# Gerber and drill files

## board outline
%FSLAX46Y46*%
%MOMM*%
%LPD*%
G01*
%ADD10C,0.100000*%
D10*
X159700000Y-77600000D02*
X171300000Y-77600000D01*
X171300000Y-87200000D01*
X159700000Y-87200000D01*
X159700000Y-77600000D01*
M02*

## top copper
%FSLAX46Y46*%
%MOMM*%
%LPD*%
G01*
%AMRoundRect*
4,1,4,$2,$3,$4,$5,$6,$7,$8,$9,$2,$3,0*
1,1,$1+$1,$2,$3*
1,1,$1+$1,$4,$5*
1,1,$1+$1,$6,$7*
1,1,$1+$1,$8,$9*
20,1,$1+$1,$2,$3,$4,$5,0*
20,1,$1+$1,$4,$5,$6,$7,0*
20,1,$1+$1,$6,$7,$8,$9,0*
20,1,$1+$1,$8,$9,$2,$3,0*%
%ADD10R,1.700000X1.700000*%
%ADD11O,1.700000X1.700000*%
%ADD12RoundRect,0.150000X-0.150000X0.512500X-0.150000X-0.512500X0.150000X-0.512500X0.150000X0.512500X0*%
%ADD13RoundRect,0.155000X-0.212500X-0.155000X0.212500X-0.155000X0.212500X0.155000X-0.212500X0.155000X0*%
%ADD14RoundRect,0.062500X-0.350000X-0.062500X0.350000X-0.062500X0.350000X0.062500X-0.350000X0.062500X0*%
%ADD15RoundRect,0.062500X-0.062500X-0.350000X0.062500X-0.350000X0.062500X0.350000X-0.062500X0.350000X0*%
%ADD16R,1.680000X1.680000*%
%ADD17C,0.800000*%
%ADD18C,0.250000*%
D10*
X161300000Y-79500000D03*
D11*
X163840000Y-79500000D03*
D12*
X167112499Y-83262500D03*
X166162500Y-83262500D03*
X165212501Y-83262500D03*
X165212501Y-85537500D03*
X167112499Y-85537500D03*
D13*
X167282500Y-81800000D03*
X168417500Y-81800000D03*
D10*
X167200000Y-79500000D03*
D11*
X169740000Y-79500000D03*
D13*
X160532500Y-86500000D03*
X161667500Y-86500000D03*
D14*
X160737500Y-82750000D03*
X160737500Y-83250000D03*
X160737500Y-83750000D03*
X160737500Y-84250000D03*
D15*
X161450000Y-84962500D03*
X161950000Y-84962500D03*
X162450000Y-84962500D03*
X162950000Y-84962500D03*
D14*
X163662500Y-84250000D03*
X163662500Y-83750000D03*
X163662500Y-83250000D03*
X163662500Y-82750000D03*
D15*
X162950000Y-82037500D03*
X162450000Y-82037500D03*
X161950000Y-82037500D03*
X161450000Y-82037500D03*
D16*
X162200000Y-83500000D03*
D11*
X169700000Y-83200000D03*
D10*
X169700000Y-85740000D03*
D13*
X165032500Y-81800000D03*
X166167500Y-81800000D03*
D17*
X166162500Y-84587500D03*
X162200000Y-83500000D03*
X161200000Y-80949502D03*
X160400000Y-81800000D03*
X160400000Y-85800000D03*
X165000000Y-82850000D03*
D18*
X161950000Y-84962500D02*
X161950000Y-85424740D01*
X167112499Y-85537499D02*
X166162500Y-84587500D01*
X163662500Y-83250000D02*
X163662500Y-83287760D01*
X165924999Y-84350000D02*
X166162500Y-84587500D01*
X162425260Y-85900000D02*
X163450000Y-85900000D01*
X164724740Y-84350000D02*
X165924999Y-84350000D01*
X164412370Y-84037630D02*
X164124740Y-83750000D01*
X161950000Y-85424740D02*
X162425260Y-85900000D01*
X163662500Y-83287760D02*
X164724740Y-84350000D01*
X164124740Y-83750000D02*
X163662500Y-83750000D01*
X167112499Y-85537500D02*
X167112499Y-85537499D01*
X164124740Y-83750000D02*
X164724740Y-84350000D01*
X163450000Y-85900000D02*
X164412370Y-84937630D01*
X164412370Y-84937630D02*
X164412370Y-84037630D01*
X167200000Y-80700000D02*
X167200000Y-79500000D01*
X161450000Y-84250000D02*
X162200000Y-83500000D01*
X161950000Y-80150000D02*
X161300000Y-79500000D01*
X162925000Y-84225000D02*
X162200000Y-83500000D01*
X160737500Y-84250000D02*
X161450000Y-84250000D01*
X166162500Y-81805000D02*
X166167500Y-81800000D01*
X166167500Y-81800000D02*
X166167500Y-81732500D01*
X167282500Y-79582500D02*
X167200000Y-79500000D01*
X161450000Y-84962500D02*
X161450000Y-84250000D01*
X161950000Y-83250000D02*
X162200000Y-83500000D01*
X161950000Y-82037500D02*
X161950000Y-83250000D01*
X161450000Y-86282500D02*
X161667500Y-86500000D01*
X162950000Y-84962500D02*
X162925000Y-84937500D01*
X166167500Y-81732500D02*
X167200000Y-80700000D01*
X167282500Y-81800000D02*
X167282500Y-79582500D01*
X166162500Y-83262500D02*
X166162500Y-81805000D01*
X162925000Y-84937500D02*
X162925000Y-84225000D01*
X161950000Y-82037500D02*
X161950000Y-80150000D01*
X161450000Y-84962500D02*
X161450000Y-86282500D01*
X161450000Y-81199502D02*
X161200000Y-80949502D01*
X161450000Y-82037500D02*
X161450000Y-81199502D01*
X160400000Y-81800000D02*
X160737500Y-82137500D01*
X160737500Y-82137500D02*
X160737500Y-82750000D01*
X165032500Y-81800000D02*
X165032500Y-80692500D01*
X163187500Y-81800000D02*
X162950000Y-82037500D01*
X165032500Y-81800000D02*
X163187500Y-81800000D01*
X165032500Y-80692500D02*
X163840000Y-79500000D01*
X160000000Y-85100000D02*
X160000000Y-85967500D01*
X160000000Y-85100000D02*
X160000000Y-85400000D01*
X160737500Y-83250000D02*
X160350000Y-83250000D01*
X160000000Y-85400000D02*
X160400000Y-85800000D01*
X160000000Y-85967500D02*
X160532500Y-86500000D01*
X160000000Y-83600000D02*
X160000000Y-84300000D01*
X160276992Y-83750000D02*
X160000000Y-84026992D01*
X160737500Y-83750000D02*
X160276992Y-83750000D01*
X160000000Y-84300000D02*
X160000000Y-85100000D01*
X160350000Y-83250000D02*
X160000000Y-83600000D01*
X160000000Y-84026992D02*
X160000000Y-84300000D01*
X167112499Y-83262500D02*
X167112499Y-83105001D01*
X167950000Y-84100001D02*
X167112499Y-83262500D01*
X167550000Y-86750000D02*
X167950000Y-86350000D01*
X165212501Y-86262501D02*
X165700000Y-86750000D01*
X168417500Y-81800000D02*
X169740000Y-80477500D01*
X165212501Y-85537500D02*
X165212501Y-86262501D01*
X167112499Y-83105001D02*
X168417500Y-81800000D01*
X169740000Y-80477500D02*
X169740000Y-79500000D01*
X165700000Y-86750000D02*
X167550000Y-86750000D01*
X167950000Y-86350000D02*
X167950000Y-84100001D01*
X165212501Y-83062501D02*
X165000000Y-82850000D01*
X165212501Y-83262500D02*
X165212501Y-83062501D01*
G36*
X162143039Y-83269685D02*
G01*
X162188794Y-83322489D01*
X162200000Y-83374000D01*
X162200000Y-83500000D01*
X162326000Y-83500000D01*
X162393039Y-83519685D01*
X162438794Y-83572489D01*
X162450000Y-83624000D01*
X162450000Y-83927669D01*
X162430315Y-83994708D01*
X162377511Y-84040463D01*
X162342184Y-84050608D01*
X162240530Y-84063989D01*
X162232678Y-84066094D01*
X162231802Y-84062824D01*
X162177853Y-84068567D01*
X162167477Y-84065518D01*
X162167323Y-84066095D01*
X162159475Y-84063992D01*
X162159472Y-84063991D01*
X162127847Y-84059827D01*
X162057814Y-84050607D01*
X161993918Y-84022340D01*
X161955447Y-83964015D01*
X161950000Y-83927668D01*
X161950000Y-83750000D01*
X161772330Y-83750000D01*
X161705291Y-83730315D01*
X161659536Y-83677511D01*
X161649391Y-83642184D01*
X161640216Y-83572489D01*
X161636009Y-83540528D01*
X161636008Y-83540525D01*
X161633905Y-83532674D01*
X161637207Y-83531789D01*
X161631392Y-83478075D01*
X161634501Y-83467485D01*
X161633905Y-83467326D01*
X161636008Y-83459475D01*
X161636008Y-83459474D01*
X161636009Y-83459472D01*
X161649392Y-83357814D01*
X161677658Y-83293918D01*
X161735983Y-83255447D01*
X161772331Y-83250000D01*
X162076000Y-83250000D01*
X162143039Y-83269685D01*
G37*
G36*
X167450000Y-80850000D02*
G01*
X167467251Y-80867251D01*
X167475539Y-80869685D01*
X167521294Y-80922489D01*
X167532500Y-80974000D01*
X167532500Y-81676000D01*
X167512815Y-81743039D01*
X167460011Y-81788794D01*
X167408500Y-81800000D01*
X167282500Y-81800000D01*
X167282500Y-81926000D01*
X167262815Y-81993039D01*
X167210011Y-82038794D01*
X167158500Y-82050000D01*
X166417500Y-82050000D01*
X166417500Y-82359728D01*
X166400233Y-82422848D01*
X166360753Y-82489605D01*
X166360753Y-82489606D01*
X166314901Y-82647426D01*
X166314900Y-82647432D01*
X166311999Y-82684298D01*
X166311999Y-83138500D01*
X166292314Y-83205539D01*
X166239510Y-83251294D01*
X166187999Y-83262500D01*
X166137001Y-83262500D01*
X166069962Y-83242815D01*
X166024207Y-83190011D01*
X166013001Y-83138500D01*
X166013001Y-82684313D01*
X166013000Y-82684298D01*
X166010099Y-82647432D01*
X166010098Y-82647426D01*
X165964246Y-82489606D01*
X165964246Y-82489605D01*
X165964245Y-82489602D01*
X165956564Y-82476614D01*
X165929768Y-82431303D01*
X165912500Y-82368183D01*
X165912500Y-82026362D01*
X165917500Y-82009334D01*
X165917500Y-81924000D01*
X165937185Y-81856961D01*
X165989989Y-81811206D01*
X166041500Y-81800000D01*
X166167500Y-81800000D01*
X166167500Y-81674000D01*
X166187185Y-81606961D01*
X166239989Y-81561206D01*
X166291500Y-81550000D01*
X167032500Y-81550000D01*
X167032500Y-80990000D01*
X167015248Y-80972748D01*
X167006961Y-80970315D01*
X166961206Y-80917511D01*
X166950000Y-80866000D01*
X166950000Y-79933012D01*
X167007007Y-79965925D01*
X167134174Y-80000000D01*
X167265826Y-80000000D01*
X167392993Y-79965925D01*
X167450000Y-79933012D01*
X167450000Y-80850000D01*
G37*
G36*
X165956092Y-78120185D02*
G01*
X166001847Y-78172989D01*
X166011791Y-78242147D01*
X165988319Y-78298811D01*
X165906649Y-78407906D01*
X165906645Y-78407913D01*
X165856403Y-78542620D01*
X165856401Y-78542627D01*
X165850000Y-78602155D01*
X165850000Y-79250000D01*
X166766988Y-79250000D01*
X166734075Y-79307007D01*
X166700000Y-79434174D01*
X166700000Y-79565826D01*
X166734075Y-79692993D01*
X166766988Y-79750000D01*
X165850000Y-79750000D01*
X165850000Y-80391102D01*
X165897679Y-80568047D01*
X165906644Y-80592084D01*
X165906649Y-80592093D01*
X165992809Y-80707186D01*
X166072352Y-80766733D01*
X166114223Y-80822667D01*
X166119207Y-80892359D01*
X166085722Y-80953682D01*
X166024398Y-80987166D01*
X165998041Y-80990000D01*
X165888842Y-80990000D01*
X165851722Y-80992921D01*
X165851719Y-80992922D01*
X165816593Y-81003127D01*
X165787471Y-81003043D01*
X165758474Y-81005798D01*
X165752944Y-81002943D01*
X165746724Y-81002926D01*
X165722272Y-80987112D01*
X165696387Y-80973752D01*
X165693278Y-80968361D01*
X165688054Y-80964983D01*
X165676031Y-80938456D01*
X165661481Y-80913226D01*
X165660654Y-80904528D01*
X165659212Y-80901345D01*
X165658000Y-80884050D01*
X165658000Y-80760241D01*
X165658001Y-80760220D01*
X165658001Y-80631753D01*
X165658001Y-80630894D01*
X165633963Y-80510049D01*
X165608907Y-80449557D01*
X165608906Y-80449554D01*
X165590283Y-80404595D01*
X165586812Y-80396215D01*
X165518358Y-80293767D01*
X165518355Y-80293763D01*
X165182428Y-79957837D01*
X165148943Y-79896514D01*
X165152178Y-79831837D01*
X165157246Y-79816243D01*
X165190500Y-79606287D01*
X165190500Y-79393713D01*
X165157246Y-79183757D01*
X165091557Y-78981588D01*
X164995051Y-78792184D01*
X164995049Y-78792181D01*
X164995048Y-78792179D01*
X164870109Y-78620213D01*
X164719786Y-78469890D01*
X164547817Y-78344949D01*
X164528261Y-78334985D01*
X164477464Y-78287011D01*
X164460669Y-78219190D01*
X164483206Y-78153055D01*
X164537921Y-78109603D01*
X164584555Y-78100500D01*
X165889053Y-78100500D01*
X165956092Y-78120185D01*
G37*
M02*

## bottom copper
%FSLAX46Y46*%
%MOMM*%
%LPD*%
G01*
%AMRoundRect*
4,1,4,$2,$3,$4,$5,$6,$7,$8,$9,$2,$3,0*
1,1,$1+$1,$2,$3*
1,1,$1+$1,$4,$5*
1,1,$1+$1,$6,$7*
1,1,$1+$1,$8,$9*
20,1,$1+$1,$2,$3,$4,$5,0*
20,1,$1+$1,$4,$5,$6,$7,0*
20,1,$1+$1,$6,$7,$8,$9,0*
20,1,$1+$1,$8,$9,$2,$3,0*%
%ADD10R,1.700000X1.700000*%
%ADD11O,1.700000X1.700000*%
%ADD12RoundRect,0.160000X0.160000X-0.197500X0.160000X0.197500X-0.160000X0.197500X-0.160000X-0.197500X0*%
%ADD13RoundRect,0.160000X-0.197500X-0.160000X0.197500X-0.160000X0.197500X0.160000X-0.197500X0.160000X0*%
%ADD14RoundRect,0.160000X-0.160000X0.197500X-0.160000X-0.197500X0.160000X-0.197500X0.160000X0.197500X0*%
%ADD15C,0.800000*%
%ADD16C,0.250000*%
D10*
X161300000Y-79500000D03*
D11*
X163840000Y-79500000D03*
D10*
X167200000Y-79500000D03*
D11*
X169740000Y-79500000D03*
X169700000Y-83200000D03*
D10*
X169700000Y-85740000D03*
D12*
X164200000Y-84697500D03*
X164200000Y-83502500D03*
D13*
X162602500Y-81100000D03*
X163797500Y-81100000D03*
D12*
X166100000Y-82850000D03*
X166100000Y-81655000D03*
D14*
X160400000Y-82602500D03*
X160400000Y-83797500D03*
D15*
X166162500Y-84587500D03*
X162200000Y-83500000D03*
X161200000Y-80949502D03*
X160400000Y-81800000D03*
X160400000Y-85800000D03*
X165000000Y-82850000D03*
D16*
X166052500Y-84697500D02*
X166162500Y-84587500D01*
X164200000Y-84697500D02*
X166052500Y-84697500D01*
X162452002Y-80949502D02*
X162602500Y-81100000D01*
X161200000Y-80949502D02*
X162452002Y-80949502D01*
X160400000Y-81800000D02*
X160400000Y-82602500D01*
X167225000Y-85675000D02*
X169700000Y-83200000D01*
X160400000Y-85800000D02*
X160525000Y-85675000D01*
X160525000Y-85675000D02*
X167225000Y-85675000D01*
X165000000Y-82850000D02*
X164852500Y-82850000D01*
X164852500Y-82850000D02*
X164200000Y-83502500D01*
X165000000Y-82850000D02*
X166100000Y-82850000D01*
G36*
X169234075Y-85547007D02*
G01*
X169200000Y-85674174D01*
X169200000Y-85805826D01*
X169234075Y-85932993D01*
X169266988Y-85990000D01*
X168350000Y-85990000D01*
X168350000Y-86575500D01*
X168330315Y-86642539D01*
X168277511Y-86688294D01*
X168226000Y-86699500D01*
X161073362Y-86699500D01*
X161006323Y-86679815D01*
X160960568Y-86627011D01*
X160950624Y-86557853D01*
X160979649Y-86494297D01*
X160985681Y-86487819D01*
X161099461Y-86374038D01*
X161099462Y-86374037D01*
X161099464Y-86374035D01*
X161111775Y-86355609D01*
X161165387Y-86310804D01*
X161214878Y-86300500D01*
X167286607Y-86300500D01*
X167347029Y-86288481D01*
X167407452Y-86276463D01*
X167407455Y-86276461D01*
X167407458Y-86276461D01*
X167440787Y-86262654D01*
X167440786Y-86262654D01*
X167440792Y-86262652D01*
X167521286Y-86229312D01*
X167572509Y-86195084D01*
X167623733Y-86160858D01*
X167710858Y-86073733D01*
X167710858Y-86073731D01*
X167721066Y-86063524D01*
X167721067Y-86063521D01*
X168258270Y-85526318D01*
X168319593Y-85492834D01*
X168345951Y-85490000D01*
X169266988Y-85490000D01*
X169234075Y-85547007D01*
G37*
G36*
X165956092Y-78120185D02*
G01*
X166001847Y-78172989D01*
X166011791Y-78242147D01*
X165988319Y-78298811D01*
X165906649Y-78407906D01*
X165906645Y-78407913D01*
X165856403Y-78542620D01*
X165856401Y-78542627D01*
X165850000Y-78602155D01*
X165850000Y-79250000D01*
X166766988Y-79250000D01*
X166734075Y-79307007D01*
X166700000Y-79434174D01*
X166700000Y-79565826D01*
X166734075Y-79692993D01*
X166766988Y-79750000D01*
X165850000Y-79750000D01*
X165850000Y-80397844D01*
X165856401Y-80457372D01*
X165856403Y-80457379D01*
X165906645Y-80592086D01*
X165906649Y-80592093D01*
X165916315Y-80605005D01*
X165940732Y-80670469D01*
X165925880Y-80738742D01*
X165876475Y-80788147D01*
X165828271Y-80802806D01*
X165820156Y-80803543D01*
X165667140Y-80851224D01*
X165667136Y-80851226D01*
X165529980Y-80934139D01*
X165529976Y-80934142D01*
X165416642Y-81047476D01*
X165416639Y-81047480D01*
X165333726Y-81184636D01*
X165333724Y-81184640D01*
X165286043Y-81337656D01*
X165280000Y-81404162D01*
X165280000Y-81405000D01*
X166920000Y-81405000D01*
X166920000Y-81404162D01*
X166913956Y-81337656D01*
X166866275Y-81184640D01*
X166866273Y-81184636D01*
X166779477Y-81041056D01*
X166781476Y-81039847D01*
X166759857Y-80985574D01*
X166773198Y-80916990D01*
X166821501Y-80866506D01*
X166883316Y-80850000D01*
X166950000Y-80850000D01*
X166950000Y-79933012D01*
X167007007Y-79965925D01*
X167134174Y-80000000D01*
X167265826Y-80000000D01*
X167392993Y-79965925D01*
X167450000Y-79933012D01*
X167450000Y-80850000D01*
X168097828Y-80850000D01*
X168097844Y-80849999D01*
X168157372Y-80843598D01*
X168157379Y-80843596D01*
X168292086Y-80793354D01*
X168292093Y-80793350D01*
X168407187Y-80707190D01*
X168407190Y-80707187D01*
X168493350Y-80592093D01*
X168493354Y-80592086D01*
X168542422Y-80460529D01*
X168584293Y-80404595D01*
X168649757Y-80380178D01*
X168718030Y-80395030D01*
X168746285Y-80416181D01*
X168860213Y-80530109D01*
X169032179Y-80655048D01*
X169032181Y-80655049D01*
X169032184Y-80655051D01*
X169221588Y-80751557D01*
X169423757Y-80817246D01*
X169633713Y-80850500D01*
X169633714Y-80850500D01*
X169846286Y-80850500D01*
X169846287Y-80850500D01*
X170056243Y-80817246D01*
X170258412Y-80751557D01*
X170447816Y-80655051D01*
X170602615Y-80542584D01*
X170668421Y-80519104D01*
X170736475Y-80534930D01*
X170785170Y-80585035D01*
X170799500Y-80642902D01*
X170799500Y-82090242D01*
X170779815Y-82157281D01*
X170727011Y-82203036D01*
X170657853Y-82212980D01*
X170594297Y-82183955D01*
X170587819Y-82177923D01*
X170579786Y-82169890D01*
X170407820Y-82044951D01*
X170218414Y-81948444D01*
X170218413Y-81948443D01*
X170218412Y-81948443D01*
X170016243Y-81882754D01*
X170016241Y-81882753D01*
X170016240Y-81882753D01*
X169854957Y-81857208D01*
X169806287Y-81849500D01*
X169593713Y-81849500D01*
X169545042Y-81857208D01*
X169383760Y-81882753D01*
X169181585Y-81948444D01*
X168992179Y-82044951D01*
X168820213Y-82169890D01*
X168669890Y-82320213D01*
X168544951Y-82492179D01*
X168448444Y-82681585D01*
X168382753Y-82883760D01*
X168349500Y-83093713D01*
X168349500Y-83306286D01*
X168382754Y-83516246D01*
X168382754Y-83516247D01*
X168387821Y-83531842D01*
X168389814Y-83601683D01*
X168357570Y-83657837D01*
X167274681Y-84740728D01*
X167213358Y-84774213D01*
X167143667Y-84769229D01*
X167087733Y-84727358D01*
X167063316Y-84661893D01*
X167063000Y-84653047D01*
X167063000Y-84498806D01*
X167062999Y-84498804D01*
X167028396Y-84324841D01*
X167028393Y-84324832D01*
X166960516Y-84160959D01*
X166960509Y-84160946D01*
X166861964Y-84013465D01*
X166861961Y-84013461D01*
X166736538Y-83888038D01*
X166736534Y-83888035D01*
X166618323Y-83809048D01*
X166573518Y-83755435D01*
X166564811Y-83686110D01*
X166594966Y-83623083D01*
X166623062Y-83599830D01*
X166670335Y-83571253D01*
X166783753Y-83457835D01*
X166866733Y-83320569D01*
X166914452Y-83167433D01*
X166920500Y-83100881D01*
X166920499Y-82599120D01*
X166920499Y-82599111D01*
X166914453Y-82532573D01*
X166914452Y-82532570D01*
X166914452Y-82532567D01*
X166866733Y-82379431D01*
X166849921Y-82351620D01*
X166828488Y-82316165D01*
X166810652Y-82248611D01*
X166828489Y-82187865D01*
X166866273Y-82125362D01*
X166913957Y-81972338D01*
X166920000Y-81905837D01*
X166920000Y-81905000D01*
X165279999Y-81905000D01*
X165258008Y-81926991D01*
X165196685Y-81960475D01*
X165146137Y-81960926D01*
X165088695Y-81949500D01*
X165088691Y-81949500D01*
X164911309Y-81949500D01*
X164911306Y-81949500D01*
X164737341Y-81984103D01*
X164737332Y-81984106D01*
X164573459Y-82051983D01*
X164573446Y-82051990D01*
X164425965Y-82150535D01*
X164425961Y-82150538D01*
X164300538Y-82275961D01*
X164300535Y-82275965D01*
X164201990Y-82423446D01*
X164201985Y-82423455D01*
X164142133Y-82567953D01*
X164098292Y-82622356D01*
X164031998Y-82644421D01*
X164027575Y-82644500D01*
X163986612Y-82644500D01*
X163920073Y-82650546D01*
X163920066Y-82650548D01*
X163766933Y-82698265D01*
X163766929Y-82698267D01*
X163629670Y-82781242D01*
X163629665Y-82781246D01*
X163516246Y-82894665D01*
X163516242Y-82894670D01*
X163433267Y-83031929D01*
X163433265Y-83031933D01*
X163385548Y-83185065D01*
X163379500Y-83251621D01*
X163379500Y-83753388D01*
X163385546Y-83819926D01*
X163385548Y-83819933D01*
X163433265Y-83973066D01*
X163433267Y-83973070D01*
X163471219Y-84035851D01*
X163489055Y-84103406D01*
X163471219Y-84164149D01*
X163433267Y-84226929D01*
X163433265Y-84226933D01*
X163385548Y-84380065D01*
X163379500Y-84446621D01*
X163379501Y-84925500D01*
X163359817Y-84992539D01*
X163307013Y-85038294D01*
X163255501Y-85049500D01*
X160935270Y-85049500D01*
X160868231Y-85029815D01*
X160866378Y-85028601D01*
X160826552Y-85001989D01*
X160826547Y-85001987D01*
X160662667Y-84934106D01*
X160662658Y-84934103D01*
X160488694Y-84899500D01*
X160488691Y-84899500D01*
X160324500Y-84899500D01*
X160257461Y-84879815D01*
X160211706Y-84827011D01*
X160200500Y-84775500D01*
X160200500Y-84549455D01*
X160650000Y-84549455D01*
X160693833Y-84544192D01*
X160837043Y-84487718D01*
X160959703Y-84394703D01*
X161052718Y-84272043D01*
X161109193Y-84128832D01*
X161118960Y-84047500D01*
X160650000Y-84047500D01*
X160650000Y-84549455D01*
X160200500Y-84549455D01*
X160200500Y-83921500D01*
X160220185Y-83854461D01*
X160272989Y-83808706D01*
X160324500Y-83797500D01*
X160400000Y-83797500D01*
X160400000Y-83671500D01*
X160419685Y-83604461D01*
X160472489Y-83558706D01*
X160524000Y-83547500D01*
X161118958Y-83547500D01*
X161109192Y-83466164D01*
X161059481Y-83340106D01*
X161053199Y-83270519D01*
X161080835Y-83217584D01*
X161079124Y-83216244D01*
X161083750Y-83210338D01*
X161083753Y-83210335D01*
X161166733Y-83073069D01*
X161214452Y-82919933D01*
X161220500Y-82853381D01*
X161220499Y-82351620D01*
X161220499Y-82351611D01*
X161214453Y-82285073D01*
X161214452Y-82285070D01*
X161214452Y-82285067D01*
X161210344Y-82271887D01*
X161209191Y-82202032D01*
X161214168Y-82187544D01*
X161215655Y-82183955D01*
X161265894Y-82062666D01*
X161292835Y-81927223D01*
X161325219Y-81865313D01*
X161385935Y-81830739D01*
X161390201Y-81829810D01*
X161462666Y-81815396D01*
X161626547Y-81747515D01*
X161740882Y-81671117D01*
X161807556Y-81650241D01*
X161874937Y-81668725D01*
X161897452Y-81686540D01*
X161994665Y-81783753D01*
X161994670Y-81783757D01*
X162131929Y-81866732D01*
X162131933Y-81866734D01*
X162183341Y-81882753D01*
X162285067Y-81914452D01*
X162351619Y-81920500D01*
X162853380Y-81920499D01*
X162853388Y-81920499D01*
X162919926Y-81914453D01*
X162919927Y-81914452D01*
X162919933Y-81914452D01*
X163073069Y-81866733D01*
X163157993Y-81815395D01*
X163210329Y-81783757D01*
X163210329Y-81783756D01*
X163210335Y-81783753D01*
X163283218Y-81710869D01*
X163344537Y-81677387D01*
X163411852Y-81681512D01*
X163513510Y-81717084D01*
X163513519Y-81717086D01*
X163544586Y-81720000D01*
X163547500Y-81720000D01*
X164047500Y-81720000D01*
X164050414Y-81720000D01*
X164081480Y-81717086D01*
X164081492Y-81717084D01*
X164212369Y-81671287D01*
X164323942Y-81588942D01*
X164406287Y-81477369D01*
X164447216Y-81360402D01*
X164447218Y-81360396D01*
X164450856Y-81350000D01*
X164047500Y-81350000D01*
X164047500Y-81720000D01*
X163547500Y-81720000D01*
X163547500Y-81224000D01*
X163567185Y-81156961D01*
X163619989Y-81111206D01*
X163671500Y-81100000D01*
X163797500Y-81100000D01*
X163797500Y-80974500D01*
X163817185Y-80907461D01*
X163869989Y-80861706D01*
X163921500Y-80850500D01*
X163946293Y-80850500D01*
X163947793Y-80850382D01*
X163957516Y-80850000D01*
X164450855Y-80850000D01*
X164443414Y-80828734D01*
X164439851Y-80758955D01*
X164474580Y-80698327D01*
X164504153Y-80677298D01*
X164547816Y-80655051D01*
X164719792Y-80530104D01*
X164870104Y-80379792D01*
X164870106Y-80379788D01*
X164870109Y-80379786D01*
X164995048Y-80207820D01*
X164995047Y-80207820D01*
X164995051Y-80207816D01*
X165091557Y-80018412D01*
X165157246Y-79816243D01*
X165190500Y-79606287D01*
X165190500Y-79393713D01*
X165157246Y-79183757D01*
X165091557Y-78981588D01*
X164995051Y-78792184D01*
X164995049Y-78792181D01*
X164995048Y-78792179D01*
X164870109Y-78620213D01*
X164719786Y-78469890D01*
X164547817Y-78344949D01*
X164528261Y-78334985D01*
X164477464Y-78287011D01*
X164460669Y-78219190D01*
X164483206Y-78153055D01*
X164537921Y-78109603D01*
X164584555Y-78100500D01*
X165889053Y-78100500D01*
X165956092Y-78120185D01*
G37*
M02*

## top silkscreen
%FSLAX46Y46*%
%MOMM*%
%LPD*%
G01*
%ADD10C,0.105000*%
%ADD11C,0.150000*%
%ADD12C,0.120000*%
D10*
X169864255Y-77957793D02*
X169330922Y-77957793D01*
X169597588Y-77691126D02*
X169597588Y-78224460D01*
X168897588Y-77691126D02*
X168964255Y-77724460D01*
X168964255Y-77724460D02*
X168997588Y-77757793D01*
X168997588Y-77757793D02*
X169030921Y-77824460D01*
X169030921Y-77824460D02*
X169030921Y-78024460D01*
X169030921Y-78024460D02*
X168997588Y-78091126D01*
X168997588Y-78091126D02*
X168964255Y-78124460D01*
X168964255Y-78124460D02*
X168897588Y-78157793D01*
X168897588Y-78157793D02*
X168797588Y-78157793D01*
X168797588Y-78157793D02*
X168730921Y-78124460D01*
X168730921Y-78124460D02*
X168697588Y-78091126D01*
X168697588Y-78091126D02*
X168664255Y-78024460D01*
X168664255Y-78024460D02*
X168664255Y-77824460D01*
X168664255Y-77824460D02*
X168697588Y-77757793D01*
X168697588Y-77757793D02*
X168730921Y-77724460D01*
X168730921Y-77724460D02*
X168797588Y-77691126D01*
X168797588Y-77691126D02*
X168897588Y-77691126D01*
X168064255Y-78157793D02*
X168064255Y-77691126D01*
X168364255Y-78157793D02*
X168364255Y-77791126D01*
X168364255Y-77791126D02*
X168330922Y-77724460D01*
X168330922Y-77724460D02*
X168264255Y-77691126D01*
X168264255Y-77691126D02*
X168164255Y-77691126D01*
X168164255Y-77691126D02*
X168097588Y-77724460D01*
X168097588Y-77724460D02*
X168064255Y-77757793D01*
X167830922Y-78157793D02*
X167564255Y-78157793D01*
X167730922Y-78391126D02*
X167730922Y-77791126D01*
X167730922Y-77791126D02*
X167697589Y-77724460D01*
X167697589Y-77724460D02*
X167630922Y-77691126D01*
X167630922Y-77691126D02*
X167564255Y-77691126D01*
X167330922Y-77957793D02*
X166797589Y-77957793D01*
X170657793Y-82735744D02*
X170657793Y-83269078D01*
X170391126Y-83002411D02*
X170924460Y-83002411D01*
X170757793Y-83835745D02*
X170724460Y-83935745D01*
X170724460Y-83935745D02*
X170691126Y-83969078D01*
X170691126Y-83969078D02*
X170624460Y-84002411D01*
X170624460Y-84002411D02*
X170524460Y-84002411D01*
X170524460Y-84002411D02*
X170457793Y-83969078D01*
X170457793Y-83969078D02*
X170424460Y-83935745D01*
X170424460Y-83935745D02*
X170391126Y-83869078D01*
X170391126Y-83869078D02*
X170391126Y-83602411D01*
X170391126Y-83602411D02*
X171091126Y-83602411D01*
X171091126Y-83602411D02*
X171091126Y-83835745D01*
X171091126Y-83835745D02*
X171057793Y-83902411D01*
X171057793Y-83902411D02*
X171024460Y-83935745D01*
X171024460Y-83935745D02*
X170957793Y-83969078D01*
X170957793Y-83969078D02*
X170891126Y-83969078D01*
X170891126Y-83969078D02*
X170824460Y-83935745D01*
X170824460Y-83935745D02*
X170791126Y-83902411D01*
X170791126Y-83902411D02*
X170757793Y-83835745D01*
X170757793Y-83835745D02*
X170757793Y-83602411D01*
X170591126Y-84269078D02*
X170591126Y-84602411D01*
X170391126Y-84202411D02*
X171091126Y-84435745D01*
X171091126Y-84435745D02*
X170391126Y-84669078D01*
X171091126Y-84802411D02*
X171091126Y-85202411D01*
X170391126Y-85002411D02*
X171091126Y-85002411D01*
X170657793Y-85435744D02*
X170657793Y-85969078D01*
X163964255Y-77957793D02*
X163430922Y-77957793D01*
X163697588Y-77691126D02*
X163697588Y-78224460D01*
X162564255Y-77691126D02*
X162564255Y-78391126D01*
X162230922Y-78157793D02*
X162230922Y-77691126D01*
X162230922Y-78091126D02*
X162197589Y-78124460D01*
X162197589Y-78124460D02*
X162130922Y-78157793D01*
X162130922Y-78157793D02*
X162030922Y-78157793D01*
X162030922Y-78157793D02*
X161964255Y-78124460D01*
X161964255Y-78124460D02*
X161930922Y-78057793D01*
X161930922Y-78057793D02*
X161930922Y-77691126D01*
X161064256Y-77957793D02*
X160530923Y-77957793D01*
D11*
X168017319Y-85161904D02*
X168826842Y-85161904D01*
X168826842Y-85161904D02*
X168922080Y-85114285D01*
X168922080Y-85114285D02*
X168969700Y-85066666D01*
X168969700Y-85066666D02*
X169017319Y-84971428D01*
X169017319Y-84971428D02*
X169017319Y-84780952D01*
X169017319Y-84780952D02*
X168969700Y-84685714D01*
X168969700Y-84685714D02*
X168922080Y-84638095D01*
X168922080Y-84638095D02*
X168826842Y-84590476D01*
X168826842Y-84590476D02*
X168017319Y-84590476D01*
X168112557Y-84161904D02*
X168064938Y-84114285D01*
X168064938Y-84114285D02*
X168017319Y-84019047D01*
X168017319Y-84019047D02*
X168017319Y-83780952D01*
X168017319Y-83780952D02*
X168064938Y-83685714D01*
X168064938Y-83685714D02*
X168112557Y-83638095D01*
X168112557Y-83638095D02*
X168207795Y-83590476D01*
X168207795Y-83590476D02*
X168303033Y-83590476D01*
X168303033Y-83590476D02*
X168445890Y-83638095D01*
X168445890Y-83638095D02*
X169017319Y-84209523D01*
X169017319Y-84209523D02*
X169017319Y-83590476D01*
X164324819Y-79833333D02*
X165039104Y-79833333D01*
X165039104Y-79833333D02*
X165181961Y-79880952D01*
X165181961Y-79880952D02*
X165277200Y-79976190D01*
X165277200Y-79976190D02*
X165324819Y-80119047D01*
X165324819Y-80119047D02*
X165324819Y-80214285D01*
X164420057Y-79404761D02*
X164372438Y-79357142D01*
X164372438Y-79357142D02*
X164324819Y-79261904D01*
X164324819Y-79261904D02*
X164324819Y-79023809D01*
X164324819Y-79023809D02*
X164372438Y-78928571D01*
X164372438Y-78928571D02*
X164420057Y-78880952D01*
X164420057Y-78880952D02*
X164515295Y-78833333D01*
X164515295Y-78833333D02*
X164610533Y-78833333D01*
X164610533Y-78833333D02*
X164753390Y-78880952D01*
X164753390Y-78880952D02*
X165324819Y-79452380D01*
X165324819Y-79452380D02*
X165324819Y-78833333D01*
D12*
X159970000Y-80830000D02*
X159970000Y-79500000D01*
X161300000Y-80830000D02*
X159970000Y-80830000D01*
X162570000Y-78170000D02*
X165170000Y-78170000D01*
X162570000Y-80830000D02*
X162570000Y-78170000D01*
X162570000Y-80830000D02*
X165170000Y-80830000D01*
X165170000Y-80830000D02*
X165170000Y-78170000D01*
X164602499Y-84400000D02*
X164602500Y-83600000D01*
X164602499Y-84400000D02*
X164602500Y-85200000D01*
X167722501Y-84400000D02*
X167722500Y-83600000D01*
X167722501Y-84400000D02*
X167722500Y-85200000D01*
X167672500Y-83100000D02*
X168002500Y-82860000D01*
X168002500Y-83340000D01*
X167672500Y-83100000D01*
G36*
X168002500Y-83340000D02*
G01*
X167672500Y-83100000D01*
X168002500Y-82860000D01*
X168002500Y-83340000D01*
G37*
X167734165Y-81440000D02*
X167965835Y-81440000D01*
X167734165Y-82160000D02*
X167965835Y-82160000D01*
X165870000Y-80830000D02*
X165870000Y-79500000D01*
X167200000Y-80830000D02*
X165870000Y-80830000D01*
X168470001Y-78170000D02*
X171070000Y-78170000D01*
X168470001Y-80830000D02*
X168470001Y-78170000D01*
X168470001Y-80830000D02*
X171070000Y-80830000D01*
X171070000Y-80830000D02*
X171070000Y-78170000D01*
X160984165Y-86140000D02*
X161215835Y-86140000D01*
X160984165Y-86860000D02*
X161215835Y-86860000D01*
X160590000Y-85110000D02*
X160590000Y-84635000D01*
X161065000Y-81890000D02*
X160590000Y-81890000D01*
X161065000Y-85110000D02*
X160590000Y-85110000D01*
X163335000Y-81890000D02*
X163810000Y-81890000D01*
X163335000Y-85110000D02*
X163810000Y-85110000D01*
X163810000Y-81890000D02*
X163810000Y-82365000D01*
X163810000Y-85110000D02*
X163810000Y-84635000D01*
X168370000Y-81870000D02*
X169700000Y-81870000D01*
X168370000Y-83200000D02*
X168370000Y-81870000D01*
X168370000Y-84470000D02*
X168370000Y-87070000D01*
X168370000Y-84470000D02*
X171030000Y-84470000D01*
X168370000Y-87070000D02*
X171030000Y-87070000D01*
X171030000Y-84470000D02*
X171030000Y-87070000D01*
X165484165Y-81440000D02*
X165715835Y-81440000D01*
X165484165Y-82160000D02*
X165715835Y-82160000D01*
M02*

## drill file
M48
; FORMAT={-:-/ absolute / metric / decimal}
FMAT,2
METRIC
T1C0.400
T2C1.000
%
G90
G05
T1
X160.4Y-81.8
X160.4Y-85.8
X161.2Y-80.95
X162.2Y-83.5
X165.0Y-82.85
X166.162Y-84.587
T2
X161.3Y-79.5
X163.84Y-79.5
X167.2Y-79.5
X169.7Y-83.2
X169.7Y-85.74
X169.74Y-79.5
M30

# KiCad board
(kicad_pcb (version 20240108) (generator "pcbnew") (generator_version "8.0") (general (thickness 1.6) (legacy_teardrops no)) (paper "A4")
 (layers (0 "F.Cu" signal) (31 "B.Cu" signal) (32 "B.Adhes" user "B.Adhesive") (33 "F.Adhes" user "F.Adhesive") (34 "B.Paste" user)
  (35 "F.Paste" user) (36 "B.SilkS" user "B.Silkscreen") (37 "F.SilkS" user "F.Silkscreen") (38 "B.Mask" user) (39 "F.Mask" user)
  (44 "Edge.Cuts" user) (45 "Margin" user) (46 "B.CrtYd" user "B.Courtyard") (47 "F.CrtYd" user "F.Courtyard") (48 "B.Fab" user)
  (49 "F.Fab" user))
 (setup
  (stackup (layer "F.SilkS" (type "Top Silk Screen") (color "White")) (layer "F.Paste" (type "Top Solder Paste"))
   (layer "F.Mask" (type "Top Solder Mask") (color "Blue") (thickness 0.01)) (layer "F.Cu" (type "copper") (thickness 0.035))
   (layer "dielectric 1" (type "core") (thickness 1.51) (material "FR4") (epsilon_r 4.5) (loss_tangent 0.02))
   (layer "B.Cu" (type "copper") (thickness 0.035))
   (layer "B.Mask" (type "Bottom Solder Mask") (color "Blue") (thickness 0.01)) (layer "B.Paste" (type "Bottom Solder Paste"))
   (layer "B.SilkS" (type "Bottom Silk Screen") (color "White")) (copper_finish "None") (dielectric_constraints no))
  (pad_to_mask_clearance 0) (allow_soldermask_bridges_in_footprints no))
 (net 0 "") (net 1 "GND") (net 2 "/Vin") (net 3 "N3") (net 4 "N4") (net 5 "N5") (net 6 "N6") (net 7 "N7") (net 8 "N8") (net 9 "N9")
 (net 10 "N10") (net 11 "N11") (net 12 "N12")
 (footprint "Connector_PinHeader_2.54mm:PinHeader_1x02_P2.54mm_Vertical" (layer "F.Cu") (at 161.3 79.5 90)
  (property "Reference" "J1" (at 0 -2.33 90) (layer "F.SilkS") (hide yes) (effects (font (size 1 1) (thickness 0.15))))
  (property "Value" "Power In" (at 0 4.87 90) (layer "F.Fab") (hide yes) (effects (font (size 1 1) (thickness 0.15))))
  (fp_line (start -1.33 -1.33) (end 0 -1.33) (stroke (width 0.12) (type solid)) (layer "F.SilkS"))
  (fp_line (start -1.33 0) (end -1.33 -1.33) (stroke (width 0.12) (type solid)) (layer "F.SilkS"))
  (fp_line (start 1.33 1.27) (end 1.33 3.87) (stroke (width 0.12) (type solid)) (layer "F.SilkS"))
  (fp_line (start -1.33 1.27) (end 1.33 1.27) (stroke (width 0.12) (type solid)) (layer "F.SilkS"))
  (fp_line (start -1.33 1.27) (end -1.33 3.87) (stroke (width 0.12) (type solid)) (layer "F.SilkS"))
  (fp_line (start -1.33 3.87) (end 1.33 3.87) (stroke (width 0.12) (type solid)) (layer "F.SilkS"))
  (pad "1" thru_hole rect (at 0 0 90) (size 1.7 1.7) (drill 1) (layers "*.Cu" "*.Mask") (remove_unused_layers no) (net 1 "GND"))
  (pad "2" thru_hole oval (at 0 2.54 90) (size 1.7 1.7) (drill 1) (layers "*.Cu" "*.Mask") (remove_unused_layers no) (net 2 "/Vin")))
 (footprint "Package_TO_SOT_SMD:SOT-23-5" (layer "F.Cu") (at 166.1625 84.4 -90)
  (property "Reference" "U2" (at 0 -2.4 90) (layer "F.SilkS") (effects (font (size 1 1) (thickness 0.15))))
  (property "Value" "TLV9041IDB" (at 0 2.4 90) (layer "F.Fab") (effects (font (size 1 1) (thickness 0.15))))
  (fp_line (start 0 1.560001) (end -0.8 1.56) (stroke (width 0.12) (type solid)) (layer "F.SilkS"))
  (fp_line (start 0 1.560001) (end 0.8 1.56) (stroke (width 0.12) (type solid)) (layer "F.SilkS"))
  (fp_line (start 0 -1.560001) (end -0.8 -1.56) (stroke (width 0.12) (type solid)) (layer "F.SilkS"))
  (fp_line (start 0 -1.560001) (end 0.8 -1.56) (stroke (width 0.12) (type solid)) (layer "F.SilkS"))
  (fp_poly
   (pts (xy -1.3 -1.51) (xy -1.54 -1.84) (xy -1.06 -1.84) (xy -1.3 -1.51)) (stroke (width 0.12) (type solid)) (fill solid) (layer "F.SilkS"))
  (pad "1" smd roundrect (at -1.1375 -0.949999 270) (size 1.325 0.6) (layers "F.Cu" "F.Paste" "F.Mask") (roundrect_rratio 0.25) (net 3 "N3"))
  (pad "2" smd roundrect (at -1.1375 0 270) (size 1.325 0.6) (layers "F.Cu" "F.Paste" "F.Mask") (roundrect_rratio 0.25) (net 1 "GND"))
  (pad "3" smd roundrect (at -1.1375 0.949999 270) (size 1.325 0.6) (layers "F.Cu" "F.Paste" "F.Mask") (roundrect_rratio 0.25) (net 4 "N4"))
  (pad "4" smd roundrect (at 1.1375 0.949999 270) (size 1.325 0.6) (layers "F.Cu" "F.Paste" "F.Mask") (roundrect_rratio 0.25) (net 3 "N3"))
  (pad "5" smd roundrect (at 1.1375 -0.949999 270) (size 1.325 0.6) (layers "F.Cu" "F.Paste" "F.Mask") (roundrect_rratio 0.25) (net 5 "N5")))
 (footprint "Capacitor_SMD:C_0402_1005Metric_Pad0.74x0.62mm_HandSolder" (layer "F.Cu") (at 167.85 81.8)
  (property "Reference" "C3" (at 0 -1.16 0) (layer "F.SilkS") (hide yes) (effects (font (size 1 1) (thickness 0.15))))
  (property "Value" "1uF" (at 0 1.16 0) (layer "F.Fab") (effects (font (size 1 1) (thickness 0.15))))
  (fp_line (start -0.115835 -0.36) (end 0.115835 -0.36) (stroke (width 0.12) (type solid)) (layer "F.SilkS"))
  (fp_line (start -0.115835 0.36) (end 0.115835 0.36) (stroke (width 0.12) (type solid)) (layer "F.SilkS"))
  (pad "1" smd roundrect (at -0.5675 0) (size 0.735 0.62) (layers "F.Cu" "F.Paste" "F.Mask") (roundrect_rratio 0.25) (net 1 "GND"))
  (pad "2" smd roundrect (at 0.5675 0) (size 0.735 0.62) (layers "F.Cu" "F.Paste" "F.Mask") (roundrect_rratio 0.25) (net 3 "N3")))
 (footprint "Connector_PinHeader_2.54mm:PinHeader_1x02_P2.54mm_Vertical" (layer "F.Cu") (at 167.2 79.5 90)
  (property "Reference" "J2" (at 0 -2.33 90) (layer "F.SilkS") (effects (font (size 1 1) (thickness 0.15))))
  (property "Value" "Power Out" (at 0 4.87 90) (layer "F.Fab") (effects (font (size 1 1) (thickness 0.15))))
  (fp_line (start -1.33 -1.33) (end 0 -1.33) (stroke (width 0.12) (type solid)) (layer "F.SilkS"))
  (fp_line (start -1.33 0) (end -1.33 -1.33) (stroke (width 0.12) (type solid)) (layer "F.SilkS"))
  (fp_line (start 1.33 1.270001) (end 1.33 3.87) (stroke (width 0.12) (type solid)) (layer "F.SilkS"))
  (fp_line (start -1.33 1.270001) (end 1.33 1.270001) (stroke (width 0.12) (type solid)) (layer "F.SilkS"))
  (fp_line (start -1.33 1.270001) (end -1.33 3.87) (stroke (width 0.12) (type solid)) (layer "F.SilkS"))
  (fp_line (start -1.33 3.87) (end 1.33 3.87) (stroke (width 0.12) (type solid)) (layer "F.SilkS"))
  (pad "1" thru_hole rect (at 0 0 90) (size 1.7 1.7) (drill 1) (layers "*.Cu" "*.Mask") (remove_unused_layers no) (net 1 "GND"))
  (pad "2" thru_hole oval (at 0 2.54 90) (size 1.7 1.7) (drill 1) (layers "*.Cu" "*.Mask") (remove_unused_layers no) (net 3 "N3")))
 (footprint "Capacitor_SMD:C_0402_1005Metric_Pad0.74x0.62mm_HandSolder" (layer "F.Cu") (at 161.1 86.5)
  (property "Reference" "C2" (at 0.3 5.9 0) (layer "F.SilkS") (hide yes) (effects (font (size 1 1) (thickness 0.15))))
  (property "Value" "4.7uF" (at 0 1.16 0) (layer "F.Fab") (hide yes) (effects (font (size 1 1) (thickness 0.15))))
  (fp_line (start -0.115835 -0.36) (end 0.115835 -0.36) (stroke (width 0.12) (type solid)) (layer "F.SilkS"))
  (fp_line (start -0.115835 0.36) (end 0.115835 0.36) (stroke (width 0.12) (type solid)) (layer "F.SilkS"))
  (pad "1" smd roundrect (at -0.5675 0) (size 0.735 0.62) (layers "F.Cu" "F.Paste" "F.Mask") (roundrect_rratio 0.25) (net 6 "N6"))
  (pad "2" smd roundrect (at 0.5675 0) (size 0.735 0.62) (layers "F.Cu" "F.Paste" "F.Mask") (roundrect_rratio 0.25) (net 1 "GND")))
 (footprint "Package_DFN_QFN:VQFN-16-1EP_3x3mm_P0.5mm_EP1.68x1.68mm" (layer "F.Cu") (at 162.2 83.5)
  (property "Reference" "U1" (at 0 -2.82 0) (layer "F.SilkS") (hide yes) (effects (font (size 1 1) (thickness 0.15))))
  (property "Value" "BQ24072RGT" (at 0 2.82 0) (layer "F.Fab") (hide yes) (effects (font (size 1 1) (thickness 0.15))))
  (fp_line (start -1.61 1.61) (end -1.61 1.135) (stroke (width 0.12) (type solid)) (layer "F.SilkS"))
  (fp_line (start -1.135 -1.61) (end -1.61 -1.61) (stroke (width 0.12) (type solid)) (layer "F.SilkS"))
  (fp_line (start -1.135 1.61) (end -1.61 1.61) (stroke (width 0.12) (type solid)) (layer "F.SilkS"))
  (fp_line (start 1.135 -1.61) (end 1.61 -1.61) (stroke (width 0.12) (type solid)) (layer "F.SilkS"))
  (fp_line (start 1.135 1.61) (end 1.61 1.61) (stroke (width 0.12) (type solid)) (layer "F.SilkS"))
  (fp_line (start 1.61 -1.61) (end 1.61 -1.135) (stroke (width 0.12) (type solid)) (layer "F.SilkS"))
  (fp_line (start 1.61 1.61) (end 1.61 1.135) (stroke (width 0.12) (type solid)) (layer "F.SilkS"))
  (pad "" smd roundrect (at -0.42 -0.42) (size 0.68 0.68) (layers "F.Paste") (roundrect_rratio 0.25))
  (pad "" smd roundrect (at -0.42 0.42) (size 0.68 0.68) (layers "F.Paste") (roundrect_rratio 0.25))
  (pad "" smd roundrect (at 0.42 -0.42) (size 0.68 0.68) (layers "F.Paste") (roundrect_rratio 0.25))
  (pad "" smd roundrect (at 0.42 0.42) (size 0.68 0.68) (layers "F.Paste") (roundrect_rratio 0.25))
  (pad "1" smd roundrect (at -1.4625 -0.75) (size 0.825 0.25) (layers "F.Cu" "F.Paste" "F.Mask") (roundrect_rratio 0.25) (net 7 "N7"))
  (pad "2" smd roundrect (at -1.4625 -0.25) (size 0.825 0.25) (layers "F.Cu" "F.Paste" "F.Mask") (roundrect_rratio 0.25) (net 6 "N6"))
  (pad "3" smd roundrect (at -1.4625 0.25) (size 0.825 0.25) (layers "F.Cu" "F.Paste" "F.Mask") (roundrect_rratio 0.25) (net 6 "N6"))
  (pad "4" smd roundrect (at -1.4625 0.75) (size 0.825 0.25) (layers "F.Cu" "F.Paste" "F.Mask") (roundrect_rratio 0.25) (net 1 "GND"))
  (pad "5" smd roundrect (at -0.75 1.4625) (size 0.25 0.825) (layers "F.Cu" "F.Paste" "F.Mask") (roundrect_rratio 0.25) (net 1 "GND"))
  (pad "6" smd roundrect (at -0.25 1.4625) (size 0.25 0.825) (layers "F.Cu" "F.Paste" "F.Mask") (roundrect_rratio 0.25) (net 5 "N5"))
  (pad "7" smd roundrect (at 0.25 1.4625) (size 0.25 0.825) (layers "F.Cu" "F.Paste" "F.Mask") (roundrect_rratio 0.25) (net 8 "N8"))
  (pad "8" smd roundrect (at 0.75 1.4625) (size 0.25 0.825) (layers "F.Cu" "F.Paste" "F.Mask") (roundrect_rratio 0.25) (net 1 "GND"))
  (pad "9" smd roundrect (at 1.4625 0.75) (size 0.825 0.25) (layers "F.Cu" "F.Paste" "F.Mask") (roundrect_rratio 0.25) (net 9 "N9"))
  (pad "10" smd roundrect (at 1.4625 0.25) (size 0.825 0.25) (layers "F.Cu" "F.Paste" "F.Mask") (roundrect_rratio 0.25) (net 5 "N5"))
  (pad "11" smd roundrect (at 1.4625 -0.25) (size 0.825 0.25) (layers "F.Cu" "F.Paste" "F.Mask") (roundrect_rratio 0.25) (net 5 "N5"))
  (pad "12" smd roundrect (at 1.4625 -0.75) (size 0.825 0.25) (layers "F.Cu" "F.Paste" "F.Mask") (roundrect_rratio 0.25) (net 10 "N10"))
  (pad "13" smd roundrect (at 0.75 -1.4625) (size 0.25 0.825) (layers "F.Cu" "F.Paste" "F.Mask") (roundrect_rratio 0.25) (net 2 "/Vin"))
  (pad "14" smd roundrect (at 0.25 -1.4625) (size 0.25 0.825) (layers "F.Cu" "F.Paste" "F.Mask") (roundrect_rratio 0.25) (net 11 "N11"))
  (pad "15" smd roundrect (at -0.25 -1.4625) (size 0.25 0.825) (layers "F.Cu" "F.Paste" "F.Mask") (roundrect_rratio 0.25) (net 1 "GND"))
  (pad "16" smd roundrect (at -0.75 -1.4625) (size 0.25 0.825) (layers "F.Cu" "F.Paste" "F.Mask") (roundrect_rratio 0.25) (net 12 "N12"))
  (pad "17" smd rect (at 0 0) (size 1.68 1.68) (layers "F.Cu" "F.Mask") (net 1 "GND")))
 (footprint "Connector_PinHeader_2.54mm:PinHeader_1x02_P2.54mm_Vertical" (layer "F.Cu") (at 169.7 83.2)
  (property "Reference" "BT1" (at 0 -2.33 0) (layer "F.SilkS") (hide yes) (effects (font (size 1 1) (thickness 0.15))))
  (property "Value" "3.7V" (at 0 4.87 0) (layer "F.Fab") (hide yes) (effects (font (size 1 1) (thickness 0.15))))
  (fp_line (start -1.33 -1.33) (end 0 -1.33) (stroke (width 0.12) (type solid)) (layer "F.SilkS"))
  (fp_line (start -1.33 0) (end -1.33 -1.33) (stroke (width 0.12) (type solid)) (layer "F.SilkS"))
  (fp_line (start -1.33 1.27) (end -1.33 3.87) (stroke (width 0.12) (type solid)) (layer "F.SilkS"))
  (fp_line (start -1.33 1.27) (end 1.33 1.27) (stroke (width 0.12) (type solid)) (layer "F.SilkS"))
  (fp_line (start -1.33 3.87) (end 1.33 3.87) (stroke (width 0.12) (type solid)) (layer "F.SilkS"))
  (fp_line (start 1.33 1.27) (end 1.33 3.87) (stroke (width 0.12) (type solid)) (layer "F.SilkS"))
  (pad "1" thru_hole oval (at 0 0) (size 1.7 1.7) (drill 1) (layers "*.Cu" "*.Mask") (remove_unused_layers no) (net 6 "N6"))
  (pad "2" thru_hole rect (at 0 2.54) (size 1.7 1.7) (drill 1) (layers "*.Cu" "*.Mask") (remove_unused_layers no) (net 1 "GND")))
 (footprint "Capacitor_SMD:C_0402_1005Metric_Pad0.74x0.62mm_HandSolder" (layer "F.Cu") (at 165.6 81.8)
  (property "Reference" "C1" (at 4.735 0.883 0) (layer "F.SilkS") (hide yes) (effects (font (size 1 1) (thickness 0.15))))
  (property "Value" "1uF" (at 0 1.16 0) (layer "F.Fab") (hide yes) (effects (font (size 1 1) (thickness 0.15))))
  (fp_line (start -0.115835 -0.36) (end 0.115835 -0.36) (stroke (width 0.12) (type solid)) (layer "F.SilkS"))
  (fp_line (start -0.115835 0.36) (end 0.115835 0.36) (stroke (width 0.12) (type solid)) (layer "F.SilkS"))
  (pad "1" smd roundrect (at -0.5675 0) (size 0.735 0.62) (layers "F.Cu" "F.Paste" "F.Mask") (roundrect_rratio 0.25) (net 2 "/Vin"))
  (pad "2" smd roundrect (at 0.5675 0) (size 0.735 0.62) (layers "F.Cu" "F.Paste" "F.Mask") (roundrect_rratio 0.25) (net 1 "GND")))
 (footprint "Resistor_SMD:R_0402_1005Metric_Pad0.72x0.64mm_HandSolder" (layer "B.Cu") (at 164.2 84.1 90)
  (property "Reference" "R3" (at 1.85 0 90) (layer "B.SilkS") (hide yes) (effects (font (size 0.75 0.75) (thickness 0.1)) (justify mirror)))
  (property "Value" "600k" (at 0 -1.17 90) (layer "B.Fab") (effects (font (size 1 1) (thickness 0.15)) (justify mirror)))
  (pad "1" smd roundrect (at -0.5975 0 90) (size 0.715 0.64) (layers "B.Cu" "B.Paste" "B.Mask") (roundrect_rratio 0.25) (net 5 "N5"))
  (pad "2" smd roundrect (at 0.5975 0 90) (size 0.715 0.64) (layers "B.Cu" "B.Paste" "B.Mask") (roundrect_rratio 0.25) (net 4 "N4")))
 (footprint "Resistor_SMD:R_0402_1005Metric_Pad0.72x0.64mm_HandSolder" (layer "B.Cu") (at 163.2 81.1)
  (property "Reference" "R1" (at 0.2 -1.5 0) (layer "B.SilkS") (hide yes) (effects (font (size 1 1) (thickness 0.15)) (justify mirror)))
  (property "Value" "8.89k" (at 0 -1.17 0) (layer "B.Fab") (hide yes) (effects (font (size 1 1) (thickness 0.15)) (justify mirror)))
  (pad "1" smd roundrect (at -0.5975 0) (size 0.715 0.64) (layers "B.Cu" "B.Paste" "B.Mask") (roundrect_rratio 0.25) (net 12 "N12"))
  (pad "2" smd roundrect (at 0.5975 0) (size 0.715 0.64) (layers "B.Cu" "B.Paste" "B.Mask") (roundrect_rratio 0.25) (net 1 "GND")
   (zone_connect 1) (thermal_bridge_width 0.5) (thermal_gap 0.3)))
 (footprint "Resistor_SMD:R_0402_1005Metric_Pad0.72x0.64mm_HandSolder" (layer "B.Cu") (at 166.1 82.2525 90)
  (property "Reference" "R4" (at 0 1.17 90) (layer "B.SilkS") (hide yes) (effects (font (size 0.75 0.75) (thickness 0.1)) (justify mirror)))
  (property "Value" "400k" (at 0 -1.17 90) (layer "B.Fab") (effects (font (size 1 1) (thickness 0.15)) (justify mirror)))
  (pad "1" smd roundrect (at -0.5975 0 90) (size 0.715 0.64) (layers "B.Cu" "B.Paste" "B.Mask") (roundrect_rratio 0.25) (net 4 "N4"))
  (pad "2" smd roundrect (at 0.5975 0 90) (size 0.715 0.64) (layers "B.Cu" "B.Paste" "B.Mask") (roundrect_rratio 0.25) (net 1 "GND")))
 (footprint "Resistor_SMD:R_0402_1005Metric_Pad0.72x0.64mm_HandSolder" (layer "B.Cu") (at 160.4 83.2 -90)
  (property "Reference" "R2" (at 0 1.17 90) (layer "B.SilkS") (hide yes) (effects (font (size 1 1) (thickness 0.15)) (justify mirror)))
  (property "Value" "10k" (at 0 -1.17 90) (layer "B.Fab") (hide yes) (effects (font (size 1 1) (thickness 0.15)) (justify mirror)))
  (pad "1" smd roundrect (at -0.5975 0 270) (size 0.715 0.64) (layers "B.Cu" "B.Paste" "B.Mask") (roundrect_rratio 0.25) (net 7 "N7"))
  (pad "2" smd roundrect (at 0.5975 0 270) (size 0.715 0.64) (layers "B.Cu" "B.Paste" "B.Mask") (roundrect_rratio 0.25) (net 1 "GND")
   (zone_connect 1) (thermal_bridge_width 0.5) (thermal_gap 0.4)))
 (gr_rect (start 159.7 77.6) (end 171.3 87.2) (stroke (width 0.1) (type default)) (fill none) (layer "Edge.Cuts"))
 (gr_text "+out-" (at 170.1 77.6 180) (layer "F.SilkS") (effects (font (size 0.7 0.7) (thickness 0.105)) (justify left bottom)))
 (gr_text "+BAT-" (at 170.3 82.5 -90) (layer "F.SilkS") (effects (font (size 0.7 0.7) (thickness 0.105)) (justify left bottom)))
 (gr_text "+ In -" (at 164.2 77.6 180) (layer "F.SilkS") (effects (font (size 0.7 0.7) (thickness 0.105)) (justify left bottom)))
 (segment (start 161.95 84.9625) (end 161.95 85.42474) (width 0.25) (layer "F.Cu") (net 5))
 (segment (start 167.112499 85.537499) (end 166.1625 84.5875) (width 0.25) (layer "F.Cu") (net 5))
 (segment (start 163.6625 83.25) (end 163.6625 83.28776) (width 0.25) (layer "F.Cu") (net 5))
 (segment (start 165.924999 84.35) (end 166.1625 84.5875) (width 0.25) (layer "F.Cu") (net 5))
 (segment (start 162.42526 85.9) (end 163.45 85.9) (width 0.25) (layer "F.Cu") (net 5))
 (segment (start 164.72474 84.35) (end 165.924999 84.35) (width 0.25) (layer "F.Cu") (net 5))
 (segment (start 164.41237 84.03763) (end 164.12474 83.75) (width 0.25) (layer "F.Cu") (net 5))
 (segment (start 161.95 85.42474) (end 162.42526 85.9) (width 0.25) (layer "F.Cu") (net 5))
 (segment (start 163.6625 83.28776) (end 164.72474 84.35) (width 0.25) (layer "F.Cu") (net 5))
 (segment (start 164.12474 83.75) (end 163.6625 83.75) (width 0.25) (layer "F.Cu") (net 5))
 (segment (start 167.112499 85.5375) (end 167.112499 85.537499) (width 0.25) (layer "F.Cu") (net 5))
 (segment (start 164.12474 83.75) (end 164.72474 84.35) (width 0.25) (layer "F.Cu") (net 5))
 (segment (start 163.45 85.9) (end 164.41237 84.93763) (width 0.25) (layer "F.Cu") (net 5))
 (segment (start 164.41237 84.93763) (end 164.41237 84.03763) (width 0.25) (layer "F.Cu") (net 5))
 (via (at 166.1625 84.5875) (size 0.8) (drill 0.4) (layers "F.Cu" "B.Cu") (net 5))
 (segment (start 166.0525 84.6975) (end 166.1625 84.5875) (width 0.25) (layer "B.Cu") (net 5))
 (segment (start 164.2 84.6975) (end 166.0525 84.6975) (width 0.25) (layer "B.Cu") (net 5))
 (segment (start 167.2 80.7) (end 167.2 79.5) (width 0.25) (layer "F.Cu") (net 1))
 (segment (start 161.45 84.25) (end 162.2 83.5) (width 0.25) (layer "F.Cu") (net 1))
 (segment (start 161.95 80.15) (end 161.3 79.5) (width 0.25) (layer "F.Cu") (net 1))
 (segment (start 162.925 84.225) (end 162.2 83.5) (width 0.25) (layer "F.Cu") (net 1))
 (segment (start 160.7375 84.25) (end 161.45 84.25) (width 0.25) (layer "F.Cu") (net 1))
 (segment (start 166.1625 81.805) (end 166.1675 81.8) (width 0.25) (layer "F.Cu") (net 1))
 (segment (start 166.1675 81.8) (end 166.1675 81.7325) (width 0.25) (layer "F.Cu") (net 1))
 (segment (start 167.2825 79.5825) (end 167.2 79.5) (width 0.25) (layer "F.Cu") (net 1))
 (segment (start 161.45 84.9625) (end 161.45 84.25) (width 0.25) (layer "F.Cu") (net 1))
 (segment (start 161.95 83.25) (end 162.2 83.5) (width 0.25) (layer "F.Cu") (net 1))
 (segment (start 161.95 82.0375) (end 161.95 83.25) (width 0.25) (layer "F.Cu") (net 1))
 (segment (start 161.45 86.2825) (end 161.6675 86.5) (width 0.25) (layer "F.Cu") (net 1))
 (segment (start 162.95 84.9625) (end 162.925 84.9375) (width 0.25) (layer "F.Cu") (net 1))
 (segment (start 166.1675 81.7325) (end 167.2 80.7) (width 0.25) (layer "F.Cu") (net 1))
 (segment (start 167.2825 81.8) (end 167.2825 79.5825) (width 0.25) (layer "F.Cu") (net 1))
 (segment (start 166.1625 83.2625) (end 166.1625 81.805) (width 0.25) (layer "F.Cu") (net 1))
 (segment (start 162.925 84.9375) (end 162.925 84.225) (width 0.25) (layer "F.Cu") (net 1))
 (segment (start 161.95 82.0375) (end 161.95 80.15) (width 0.25) (layer "F.Cu") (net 1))
 (segment (start 161.45 84.9625) (end 161.45 86.2825) (width 0.25) (layer "F.Cu") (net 1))
 (via (at 162.2 83.5) (size 0.8) (drill 0.4) (layers "F.Cu" "B.Cu") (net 1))
 (segment (start 161.45 81.199502) (end 161.2 80.949502) (width 0.25) (layer "F.Cu") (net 12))
 (segment (start 161.45 82.0375) (end 161.45 81.199502) (width 0.25) (layer "F.Cu") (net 12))
 (via (at 161.2 80.949502) (size 0.8) (drill 0.4) (layers "F.Cu" "B.Cu") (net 12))
 (segment (start 162.452002 80.949502) (end 162.6025 81.1) (width 0.25) (layer "B.Cu") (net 12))
 (segment (start 161.2 80.949502) (end 162.452002 80.949502) (width 0.25) (layer "B.Cu") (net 12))
 (segment (start 160.4 81.8) (end 160.7375 82.1375) (width 0.25) (layer "F.Cu") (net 7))
 (segment (start 160.7375 82.1375) (end 160.7375 82.75) (width 0.25) (layer "F.Cu") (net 7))
 (via (at 160.4 81.8) (size 0.8) (drill 0.4) (layers "F.Cu" "B.Cu") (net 7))
 (segment (start 160.4 81.8) (end 160.4 82.6025) (width 0.25) (layer "B.Cu") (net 7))
 (segment (start 165.0325 81.8) (end 165.0325 80.6925) (width 0.25) (layer "F.Cu") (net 2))
 (segment (start 163.1875 81.8) (end 162.95 82.0375) (width 0.25) (layer "F.Cu") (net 2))
 (segment (start 165.0325 81.8) (end 163.1875 81.8) (width 0.25) (layer "F.Cu") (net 2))
 (segment (start 165.0325 80.6925) (end 163.84 79.5) (width 0.25) (layer "F.Cu") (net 2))
 (segment (start 160 85.1) (end 160 85.9675) (width 0.25) (layer "F.Cu") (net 6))
 (segment (start 160 85.1) (end 160 85.4) (width 0.25) (layer "F.Cu") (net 6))
 (segment (start 160.7375 83.25) (end 160.35 83.25) (width 0.25) (layer "F.Cu") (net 6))
 (segment (start 160 85.4) (end 160.4 85.8) (width 0.25) (layer "F.Cu") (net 6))
 (segment (start 160 85.9675) (end 160.5325 86.5) (width 0.25) (layer "F.Cu") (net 6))
 (segment (start 160 83.6) (end 160 84.3) (width 0.25) (layer "F.Cu") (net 6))
 (segment (start 160.276992 83.75) (end 160 84.026992) (width 0.25) (layer "F.Cu") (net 6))
 (segment (start 160.7375 83.75) (end 160.276992 83.75) (width 0.25) (layer "F.Cu") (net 6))
 (segment (start 160 84.3) (end 160 85.1) (width 0.25) (layer "F.Cu") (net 6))
 (segment (start 160.35 83.25) (end 160 83.6) (width 0.25) (layer "F.Cu") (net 6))
 (segment (start 160 84.026992) (end 160 84.3) (width 0.25) (layer "F.Cu") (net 6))
 (via (at 160.4 85.8) (size 0.8) (drill 0.4) (layers "F.Cu" "B.Cu") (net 6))
 (segment (start 167.225 85.675) (end 169.7 83.2) (width 0.25) (layer "B.Cu") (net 6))
 (segment (start 160.4 85.8) (end 160.525 85.675) (width 0.25) (layer "B.Cu") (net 6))
 (segment (start 160.525 85.675) (end 167.225 85.675) (width 0.25) (layer "B.Cu") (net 6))
 (segment (start 167.112499 83.2625) (end 167.112499 83.105001) (width 0.25) (layer "F.Cu") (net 3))
 (segment (start 167.95 84.100001) (end 167.112499 83.2625) (width 0.25) (layer "F.Cu") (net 3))
 (segment (start 167.55 86.75) (end 167.95 86.35) (width 0.25) (layer "F.Cu") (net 3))
 (segment (start 165.212501 86.262501) (end 165.7 86.75) (width 0.25) (layer "F.Cu") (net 3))
 (segment (start 168.4175 81.8) (end 169.74 80.4775) (width 0.25) (layer "F.Cu") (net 3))
 (segment (start 165.212501 85.5375) (end 165.212501 86.262501) (width 0.25) (layer "F.Cu") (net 3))
 (segment (start 167.112499 83.105001) (end 168.4175 81.8) (width 0.25) (layer "F.Cu") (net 3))
 (segment (start 169.74 80.4775) (end 169.74 79.5) (width 0.25) (layer "F.Cu") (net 3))
 (segment (start 165.7 86.75) (end 167.55 86.75) (width 0.25) (layer "F.Cu") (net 3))
 (segment (start 167.95 86.35) (end 167.95 84.100001) (width 0.25) (layer "F.Cu") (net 3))
 (segment (start 165.212501 83.062501) (end 165 82.85) (width 0.25) (layer "F.Cu") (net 4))
 (segment (start 165.212501 83.2625) (end 165.212501 83.062501) (width 0.25) (layer "F.Cu") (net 4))
 (via (at 165 82.85) (size 0.8) (drill 0.4) (layers "F.Cu" "B.Cu") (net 4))
 (segment (start 165 82.85) (end 164.8525 82.85) (width 0.25) (layer "B.Cu") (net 4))
 (segment (start 164.8525 82.85) (end 164.2 83.5025) (width 0.25) (layer "B.Cu") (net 4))
 (segment (start 165 82.85) (end 166.1 82.85) (width 0.25) (layer "B.Cu") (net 4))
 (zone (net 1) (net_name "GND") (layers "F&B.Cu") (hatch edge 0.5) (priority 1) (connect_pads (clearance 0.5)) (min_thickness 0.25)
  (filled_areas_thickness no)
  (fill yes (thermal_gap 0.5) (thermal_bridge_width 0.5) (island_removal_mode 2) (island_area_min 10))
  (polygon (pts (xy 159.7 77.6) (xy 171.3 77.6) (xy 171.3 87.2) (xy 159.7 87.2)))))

